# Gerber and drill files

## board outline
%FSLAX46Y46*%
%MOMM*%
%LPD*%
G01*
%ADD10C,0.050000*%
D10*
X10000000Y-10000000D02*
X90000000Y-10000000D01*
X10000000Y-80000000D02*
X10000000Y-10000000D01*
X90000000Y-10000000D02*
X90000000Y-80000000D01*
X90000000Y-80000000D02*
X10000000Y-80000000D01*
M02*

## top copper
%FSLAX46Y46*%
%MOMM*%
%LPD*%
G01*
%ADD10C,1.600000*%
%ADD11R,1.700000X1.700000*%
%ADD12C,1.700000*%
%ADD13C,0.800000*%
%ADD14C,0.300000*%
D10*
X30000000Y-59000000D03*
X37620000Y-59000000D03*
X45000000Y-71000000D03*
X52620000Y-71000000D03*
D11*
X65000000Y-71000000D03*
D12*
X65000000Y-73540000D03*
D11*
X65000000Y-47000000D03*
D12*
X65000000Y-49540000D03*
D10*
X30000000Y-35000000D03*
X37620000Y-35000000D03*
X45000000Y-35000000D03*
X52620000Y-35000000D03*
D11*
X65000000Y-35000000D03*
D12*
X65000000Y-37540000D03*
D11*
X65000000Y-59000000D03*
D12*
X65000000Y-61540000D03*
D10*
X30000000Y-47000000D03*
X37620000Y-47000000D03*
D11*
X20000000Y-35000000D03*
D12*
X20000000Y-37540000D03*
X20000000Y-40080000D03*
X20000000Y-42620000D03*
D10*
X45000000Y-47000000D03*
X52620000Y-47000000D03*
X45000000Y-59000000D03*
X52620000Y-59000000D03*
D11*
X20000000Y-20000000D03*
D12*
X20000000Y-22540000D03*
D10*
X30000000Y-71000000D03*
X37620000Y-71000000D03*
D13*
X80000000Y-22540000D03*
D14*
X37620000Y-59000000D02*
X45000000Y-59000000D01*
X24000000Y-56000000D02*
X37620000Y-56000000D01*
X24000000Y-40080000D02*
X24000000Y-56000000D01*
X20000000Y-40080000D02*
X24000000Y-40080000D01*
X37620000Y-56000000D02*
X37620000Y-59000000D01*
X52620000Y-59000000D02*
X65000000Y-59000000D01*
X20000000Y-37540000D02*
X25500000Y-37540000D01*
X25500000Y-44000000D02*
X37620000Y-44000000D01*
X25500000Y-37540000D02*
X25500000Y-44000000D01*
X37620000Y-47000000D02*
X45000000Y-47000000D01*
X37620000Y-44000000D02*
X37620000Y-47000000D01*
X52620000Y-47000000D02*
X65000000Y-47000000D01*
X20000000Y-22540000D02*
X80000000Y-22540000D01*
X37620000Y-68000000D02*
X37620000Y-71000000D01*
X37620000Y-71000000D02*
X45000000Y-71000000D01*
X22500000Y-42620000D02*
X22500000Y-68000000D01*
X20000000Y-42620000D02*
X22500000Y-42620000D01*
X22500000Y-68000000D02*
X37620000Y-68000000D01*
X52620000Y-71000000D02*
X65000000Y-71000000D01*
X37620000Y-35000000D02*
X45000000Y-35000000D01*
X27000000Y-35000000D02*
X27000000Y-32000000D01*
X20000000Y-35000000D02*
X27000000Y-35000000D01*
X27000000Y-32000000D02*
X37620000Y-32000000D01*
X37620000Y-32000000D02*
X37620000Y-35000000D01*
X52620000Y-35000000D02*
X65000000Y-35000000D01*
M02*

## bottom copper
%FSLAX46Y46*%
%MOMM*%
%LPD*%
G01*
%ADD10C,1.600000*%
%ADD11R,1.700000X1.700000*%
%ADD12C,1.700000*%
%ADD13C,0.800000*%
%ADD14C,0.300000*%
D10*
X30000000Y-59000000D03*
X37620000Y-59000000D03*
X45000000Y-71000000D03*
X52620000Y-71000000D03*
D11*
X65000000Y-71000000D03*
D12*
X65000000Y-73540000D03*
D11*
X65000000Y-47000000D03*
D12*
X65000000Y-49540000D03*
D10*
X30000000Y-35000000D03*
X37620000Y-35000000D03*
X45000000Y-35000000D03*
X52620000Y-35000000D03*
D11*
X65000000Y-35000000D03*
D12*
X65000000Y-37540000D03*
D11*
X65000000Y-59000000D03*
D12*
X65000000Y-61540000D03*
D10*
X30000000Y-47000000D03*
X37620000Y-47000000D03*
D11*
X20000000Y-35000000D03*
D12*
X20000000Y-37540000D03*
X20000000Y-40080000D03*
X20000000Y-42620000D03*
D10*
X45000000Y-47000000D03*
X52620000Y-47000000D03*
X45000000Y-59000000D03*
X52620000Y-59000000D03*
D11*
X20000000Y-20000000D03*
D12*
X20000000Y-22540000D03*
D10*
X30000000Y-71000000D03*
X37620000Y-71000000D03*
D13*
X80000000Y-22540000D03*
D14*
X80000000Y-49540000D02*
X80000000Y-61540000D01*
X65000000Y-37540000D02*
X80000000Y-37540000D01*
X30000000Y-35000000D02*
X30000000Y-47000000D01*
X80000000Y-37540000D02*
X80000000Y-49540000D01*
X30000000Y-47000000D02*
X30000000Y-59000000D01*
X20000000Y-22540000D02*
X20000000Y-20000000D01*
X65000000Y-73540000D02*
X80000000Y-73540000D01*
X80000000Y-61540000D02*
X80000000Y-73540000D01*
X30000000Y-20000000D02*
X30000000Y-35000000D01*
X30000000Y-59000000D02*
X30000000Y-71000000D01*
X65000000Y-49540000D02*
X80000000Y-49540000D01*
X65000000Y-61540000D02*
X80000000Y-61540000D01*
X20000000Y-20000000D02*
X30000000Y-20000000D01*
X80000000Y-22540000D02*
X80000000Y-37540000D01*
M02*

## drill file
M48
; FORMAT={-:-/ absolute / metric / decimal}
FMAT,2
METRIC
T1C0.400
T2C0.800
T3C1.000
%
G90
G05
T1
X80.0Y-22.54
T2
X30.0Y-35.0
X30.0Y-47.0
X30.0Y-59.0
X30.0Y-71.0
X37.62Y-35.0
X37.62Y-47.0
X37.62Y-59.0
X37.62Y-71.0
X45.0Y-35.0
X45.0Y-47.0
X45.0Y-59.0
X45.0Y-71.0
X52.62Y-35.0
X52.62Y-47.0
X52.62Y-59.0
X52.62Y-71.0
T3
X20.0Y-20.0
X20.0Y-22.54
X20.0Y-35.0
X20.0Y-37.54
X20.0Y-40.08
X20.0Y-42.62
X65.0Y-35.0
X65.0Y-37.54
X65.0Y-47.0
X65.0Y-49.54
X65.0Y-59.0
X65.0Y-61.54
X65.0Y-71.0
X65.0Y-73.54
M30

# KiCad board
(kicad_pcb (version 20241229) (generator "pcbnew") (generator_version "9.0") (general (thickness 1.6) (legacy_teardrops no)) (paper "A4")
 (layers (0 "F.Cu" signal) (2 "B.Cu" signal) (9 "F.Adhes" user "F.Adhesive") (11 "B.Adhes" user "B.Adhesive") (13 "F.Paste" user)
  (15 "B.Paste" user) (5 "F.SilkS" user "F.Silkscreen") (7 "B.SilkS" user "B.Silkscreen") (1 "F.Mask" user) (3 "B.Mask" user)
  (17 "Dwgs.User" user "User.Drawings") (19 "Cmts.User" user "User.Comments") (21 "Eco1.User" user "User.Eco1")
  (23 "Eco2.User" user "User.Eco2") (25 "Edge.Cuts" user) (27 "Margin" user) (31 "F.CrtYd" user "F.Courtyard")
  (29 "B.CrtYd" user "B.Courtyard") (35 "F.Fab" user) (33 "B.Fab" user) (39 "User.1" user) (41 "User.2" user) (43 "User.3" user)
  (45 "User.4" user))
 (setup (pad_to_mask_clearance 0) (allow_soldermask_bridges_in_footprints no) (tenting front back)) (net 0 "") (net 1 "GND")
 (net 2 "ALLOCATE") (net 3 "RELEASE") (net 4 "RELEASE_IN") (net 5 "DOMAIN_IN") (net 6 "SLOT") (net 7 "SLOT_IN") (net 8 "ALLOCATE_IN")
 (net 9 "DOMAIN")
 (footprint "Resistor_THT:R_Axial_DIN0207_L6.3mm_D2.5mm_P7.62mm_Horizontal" (layer "F.Cu") (at 30 59)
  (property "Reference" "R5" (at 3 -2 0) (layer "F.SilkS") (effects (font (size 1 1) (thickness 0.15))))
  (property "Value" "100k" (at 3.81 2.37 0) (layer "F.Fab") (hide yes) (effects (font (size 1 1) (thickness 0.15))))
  (pad "1" thru_hole circle (at 0 0) (size 1.6 1.6) (drill 0.8) (layers "*.Cu" "*.Mask") (remove_unused_layers no) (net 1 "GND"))
  (pad "2" thru_hole circle (at 7.62 0) (size 1.6 1.6) (drill 0.8) (layers "*.Cu" "*.Mask") (remove_unused_layers no) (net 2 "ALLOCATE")))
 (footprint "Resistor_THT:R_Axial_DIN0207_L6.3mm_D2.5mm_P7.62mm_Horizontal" (layer "F.Cu") (at 45 71)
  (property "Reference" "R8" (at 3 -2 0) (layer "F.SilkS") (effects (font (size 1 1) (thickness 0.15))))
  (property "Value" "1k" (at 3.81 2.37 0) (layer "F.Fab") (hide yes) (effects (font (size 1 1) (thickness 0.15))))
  (pad "1" thru_hole circle (at 0 0) (size 1.6 1.6) (drill 0.8) (layers "*.Cu" "*.Mask") (remove_unused_layers no) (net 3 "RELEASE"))
  (pad "2" thru_hole circle (at 7.62 0) (size 1.6 1.6) (drill 0.8) (layers "*.Cu" "*.Mask") (remove_unused_layers no) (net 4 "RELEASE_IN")))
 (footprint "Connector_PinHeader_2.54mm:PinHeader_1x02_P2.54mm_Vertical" (layer "F.Cu") (at 65 71)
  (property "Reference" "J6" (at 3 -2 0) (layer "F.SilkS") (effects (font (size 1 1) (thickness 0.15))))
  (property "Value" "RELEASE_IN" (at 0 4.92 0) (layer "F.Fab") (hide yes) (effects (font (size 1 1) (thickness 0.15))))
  (pad "1" thru_hole rect (at 0 0) (size 1.7 1.7) (drill 1) (layers "*.Cu" "*.Mask") (remove_unused_layers no) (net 4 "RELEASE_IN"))
  (pad "2" thru_hole circle (at 0 2.54) (size 1.7 1.7) (drill 1) (layers "*.Cu" "*.Mask") (remove_unused_layers no) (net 1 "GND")))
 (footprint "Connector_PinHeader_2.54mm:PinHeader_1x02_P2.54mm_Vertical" (layer "F.Cu") (at 65 47)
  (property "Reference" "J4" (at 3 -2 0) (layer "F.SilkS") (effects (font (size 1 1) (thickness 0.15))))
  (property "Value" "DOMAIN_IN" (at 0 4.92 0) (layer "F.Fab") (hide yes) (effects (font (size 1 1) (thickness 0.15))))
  (pad "1" thru_hole rect (at 0 0) (size 1.7 1.7) (drill 1) (layers "*.Cu" "*.Mask") (remove_unused_layers no) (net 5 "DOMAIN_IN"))
  (pad "2" thru_hole circle (at 0 2.54) (size 1.7 1.7) (drill 1) (layers "*.Cu" "*.Mask") (remove_unused_layers no) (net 1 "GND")))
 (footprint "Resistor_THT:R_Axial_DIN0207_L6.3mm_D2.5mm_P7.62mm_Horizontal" (layer "F.Cu") (at 30 35)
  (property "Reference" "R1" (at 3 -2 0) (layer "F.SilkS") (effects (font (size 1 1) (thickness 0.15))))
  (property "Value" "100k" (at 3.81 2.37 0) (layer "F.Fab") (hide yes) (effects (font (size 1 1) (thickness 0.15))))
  (pad "1" thru_hole circle (at 0 0) (size 1.6 1.6) (drill 0.8) (layers "*.Cu" "*.Mask") (remove_unused_layers no) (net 1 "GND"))
  (pad "2" thru_hole circle (at 7.62 0) (size 1.6 1.6) (drill 0.8) (layers "*.Cu" "*.Mask") (remove_unused_layers no) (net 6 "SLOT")))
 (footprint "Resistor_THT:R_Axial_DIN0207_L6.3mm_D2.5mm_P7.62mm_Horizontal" (layer "F.Cu") (at 45 35)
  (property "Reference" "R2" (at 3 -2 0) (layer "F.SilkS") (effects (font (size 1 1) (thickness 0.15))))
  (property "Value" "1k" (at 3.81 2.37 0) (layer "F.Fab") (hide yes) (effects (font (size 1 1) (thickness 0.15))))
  (pad "1" thru_hole circle (at 0 0) (size 1.6 1.6) (drill 0.8) (layers "*.Cu" "*.Mask") (remove_unused_layers no) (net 6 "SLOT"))
  (pad "2" thru_hole circle (at 7.62 0) (size 1.6 1.6) (drill 0.8) (layers "*.Cu" "*.Mask") (remove_unused_layers no) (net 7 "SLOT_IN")))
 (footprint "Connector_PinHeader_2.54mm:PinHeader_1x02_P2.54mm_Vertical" (layer "F.Cu") (at 65 35)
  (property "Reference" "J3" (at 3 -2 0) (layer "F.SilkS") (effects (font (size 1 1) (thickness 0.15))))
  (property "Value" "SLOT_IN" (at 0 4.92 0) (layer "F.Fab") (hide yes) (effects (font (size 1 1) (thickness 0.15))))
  (pad "1" thru_hole rect (at 0 0) (size 1.7 1.7) (drill 1) (layers "*.Cu" "*.Mask") (remove_unused_layers no) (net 7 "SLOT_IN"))
  (pad "2" thru_hole circle (at 0 2.54) (size 1.7 1.7) (drill 1) (layers "*.Cu" "*.Mask") (remove_unused_layers no) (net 1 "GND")))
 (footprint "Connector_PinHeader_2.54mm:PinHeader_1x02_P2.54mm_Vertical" (layer "F.Cu") (at 65 59)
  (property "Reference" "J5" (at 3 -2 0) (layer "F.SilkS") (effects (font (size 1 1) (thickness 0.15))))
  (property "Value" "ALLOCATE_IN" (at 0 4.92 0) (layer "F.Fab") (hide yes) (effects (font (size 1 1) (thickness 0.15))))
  (pad "1" thru_hole rect (at 0 0) (size 1.7 1.7) (drill 1) (layers "*.Cu" "*.Mask") (remove_unused_layers no) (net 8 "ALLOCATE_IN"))
  (pad "2" thru_hole circle (at 0 2.54) (size 1.7 1.7) (drill 1) (layers "*.Cu" "*.Mask") (remove_unused_layers no) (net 1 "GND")))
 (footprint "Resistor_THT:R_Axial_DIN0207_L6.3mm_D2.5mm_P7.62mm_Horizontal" (layer "F.Cu") (at 30 47)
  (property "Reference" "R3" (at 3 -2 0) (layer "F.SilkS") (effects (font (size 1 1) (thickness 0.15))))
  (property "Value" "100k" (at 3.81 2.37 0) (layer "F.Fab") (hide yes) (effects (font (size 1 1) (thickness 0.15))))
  (pad "1" thru_hole circle (at 0 0) (size 1.6 1.6) (drill 0.8) (layers "*.Cu" "*.Mask") (remove_unused_layers no) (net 1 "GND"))
  (pad "2" thru_hole circle (at 7.62 0) (size 1.6 1.6) (drill 0.8) (layers "*.Cu" "*.Mask") (remove_unused_layers no) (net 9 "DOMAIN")))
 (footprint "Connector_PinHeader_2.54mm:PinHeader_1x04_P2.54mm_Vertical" (layer "F.Cu") (at 20 35)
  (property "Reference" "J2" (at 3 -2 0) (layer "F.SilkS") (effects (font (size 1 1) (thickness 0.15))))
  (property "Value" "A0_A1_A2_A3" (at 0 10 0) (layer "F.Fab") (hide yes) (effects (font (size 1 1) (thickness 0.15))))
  (pad "1" thru_hole rect (at 0 0) (size 1.7 1.7) (drill 1) (layers "*.Cu" "*.Mask") (remove_unused_layers no) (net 6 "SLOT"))
  (pad "2" thru_hole circle (at 0 2.54) (size 1.7 1.7) (drill 1) (layers "*.Cu" "*.Mask") (remove_unused_layers no) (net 9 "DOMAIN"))
  (pad "3" thru_hole circle (at 0 5.08) (size 1.7 1.7) (drill 1) (layers "*.Cu" "*.Mask") (remove_unused_layers no) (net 2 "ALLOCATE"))
  (pad "4" thru_hole circle (at 0 7.62) (size 1.7 1.7) (drill 1) (layers "*.Cu" "*.Mask") (remove_unused_layers no) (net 3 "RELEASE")))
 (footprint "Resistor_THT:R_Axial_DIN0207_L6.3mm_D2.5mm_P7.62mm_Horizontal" (layer "F.Cu") (at 45 47)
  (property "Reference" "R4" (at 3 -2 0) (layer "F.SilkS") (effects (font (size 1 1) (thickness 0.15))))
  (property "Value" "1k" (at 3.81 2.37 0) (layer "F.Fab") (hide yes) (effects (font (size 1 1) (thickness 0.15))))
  (pad "1" thru_hole circle (at 0 0) (size 1.6 1.6) (drill 0.8) (layers "*.Cu" "*.Mask") (remove_unused_layers no) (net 9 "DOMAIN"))
  (pad "2" thru_hole circle (at 7.62 0) (size 1.6 1.6) (drill 0.8) (layers "*.Cu" "*.Mask") (remove_unused_layers no) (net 5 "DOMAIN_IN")))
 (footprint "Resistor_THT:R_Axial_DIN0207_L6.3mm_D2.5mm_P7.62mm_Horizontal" (layer "F.Cu") (at 45 59)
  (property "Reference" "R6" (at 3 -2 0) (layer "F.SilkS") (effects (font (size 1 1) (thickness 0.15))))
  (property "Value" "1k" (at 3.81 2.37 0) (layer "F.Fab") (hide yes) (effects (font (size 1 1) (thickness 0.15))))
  (pad "1" thru_hole circle (at 0 0) (size 1.6 1.6) (drill 0.8) (layers "*.Cu" "*.Mask") (remove_unused_layers no) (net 2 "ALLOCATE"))
  (pad "2" thru_hole circle (at 7.62 0) (size 1.6 1.6) (drill 0.8) (layers "*.Cu" "*.Mask") (remove_unused_layers no) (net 8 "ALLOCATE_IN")))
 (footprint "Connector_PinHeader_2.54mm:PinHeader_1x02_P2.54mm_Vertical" (layer "F.Cu") (at 20 20)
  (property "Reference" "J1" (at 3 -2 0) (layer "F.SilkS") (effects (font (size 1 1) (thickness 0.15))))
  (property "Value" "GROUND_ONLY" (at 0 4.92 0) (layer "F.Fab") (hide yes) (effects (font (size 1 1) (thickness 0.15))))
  (pad "1" thru_hole rect (at 0 0) (size 1.7 1.7) (drill 1) (layers "*.Cu" "*.Mask") (remove_unused_layers no) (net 1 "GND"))
  (pad "2" thru_hole circle (at 0 2.54) (size 1.7 1.7) (drill 1) (layers "*.Cu" "*.Mask") (remove_unused_layers no) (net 1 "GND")))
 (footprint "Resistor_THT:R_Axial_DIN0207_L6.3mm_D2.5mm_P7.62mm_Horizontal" (layer "F.Cu") (at 30 71)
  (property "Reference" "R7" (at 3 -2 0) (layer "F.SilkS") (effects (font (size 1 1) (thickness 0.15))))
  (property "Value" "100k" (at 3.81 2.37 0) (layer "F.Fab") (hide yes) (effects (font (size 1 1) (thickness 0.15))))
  (pad "1" thru_hole circle (at 0 0) (size 1.6 1.6) (drill 0.8) (layers "*.Cu" "*.Mask") (remove_unused_layers no) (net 1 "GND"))
  (pad "2" thru_hole circle (at 7.62 0) (size 1.6 1.6) (drill 0.8) (layers "*.Cu" "*.Mask") (remove_unused_layers no) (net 3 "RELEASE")))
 (gr_line (start 10 10) (end 90 10) (stroke (width 0.05) (type default)) (layer "Edge.Cuts"))
 (gr_line (start 10 80) (end 10 10) (stroke (width 0.05) (type default)) (layer "Edge.Cuts"))
 (gr_line (start 90 10) (end 90 80) (stroke (width 0.05) (type default)) (layer "Edge.Cuts"))
 (gr_line (start 90 80) (end 10 80) (stroke (width 0.05) (type default)) (layer "Edge.Cuts"))
 (segment (start 37.62 59) (end 45 59) (width 0.3) (layer "F.Cu") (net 2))
 (segment (start 24 56) (end 37.62 56) (width 0.3) (layer "F.Cu") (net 2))
 (segment (start 24 40.08) (end 24 56) (width 0.3) (layer "F.Cu") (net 2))
 (segment (start 20 40.08) (end 24 40.08) (width 0.3) (layer "F.Cu") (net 2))
 (segment (start 37.62 56) (end 37.62 59) (width 0.3) (layer "F.Cu") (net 2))
 (segment (start 52.62 59) (end 65 59) (width 0.3) (layer "F.Cu") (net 8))
 (segment (start 20 37.54) (end 25.5 37.54) (width 0.3) (layer "F.Cu") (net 9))
 (segment (start 25.5 44) (end 37.62 44) (width 0.3) (layer "F.Cu") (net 9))
 (segment (start 25.5 37.54) (end 25.5 44) (width 0.3) (layer "F.Cu") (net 9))
 (segment (start 37.62 47) (end 45 47) (width 0.3) (layer "F.Cu") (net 9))
 (segment (start 37.62 44) (end 37.62 47) (width 0.3) (layer "F.Cu") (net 9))
 (segment (start 52.62 47) (end 65 47) (width 0.3) (layer "F.Cu") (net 5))
 (segment (start 20 22.54) (end 80 22.54) (width 0.3) (layer "F.Cu") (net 1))
 (via (at 80 22.54) (size 0.8) (drill 0.4) (layers "F.Cu" "B.Cu") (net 1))
 (segment (start 80 49.54) (end 80 61.54) (width 0.3) (layer "B.Cu") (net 1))
 (segment (start 65 37.54) (end 80 37.54) (width 0.3) (layer "B.Cu") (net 1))
 (segment (start 30 35) (end 30 47) (width 0.3) (layer "B.Cu") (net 1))
 (segment (start 80 37.54) (end 80 49.54) (width 0.3) (layer "B.Cu") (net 1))
 (segment (start 30 47) (end 30 59) (width 0.3) (layer "B.Cu") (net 1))
 (segment (start 20 22.54) (end 20 20) (width 0.3) (layer "B.Cu") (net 1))
 (segment (start 65 73.54) (end 80 73.54) (width 0.3) (layer "B.Cu") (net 1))
 (segment (start 80 61.54) (end 80 73.54) (width 0.3) (layer "B.Cu") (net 1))
 (segment (start 30 20) (end 30 35) (width 0.3) (layer "B.Cu") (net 1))
 (segment (start 30 59) (end 30 71) (width 0.3) (layer "B.Cu") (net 1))
 (segment (start 65 49.54) (end 80 49.54) (width 0.3) (layer "B.Cu") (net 1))
 (segment (start 65 61.54) (end 80 61.54) (width 0.3) (layer "B.Cu") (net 1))
 (segment (start 20 20) (end 30 20) (width 0.3) (layer "B.Cu") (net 1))
 (segment (start 80 22.54) (end 80 37.54) (width 0.3) (layer "B.Cu") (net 1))
 (segment (start 37.62 68) (end 37.62 71) (width 0.3) (layer "F.Cu") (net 3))
 (segment (start 37.62 71) (end 45 71) (width 0.3) (layer "F.Cu") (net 3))
 (segment (start 22.5 42.62) (end 22.5 68) (width 0.3) (layer "F.Cu") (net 3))
 (segment (start 20 42.62) (end 22.5 42.62) (width 0.3) (layer "F.Cu") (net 3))
 (segment (start 22.5 68) (end 37.62 68) (width 0.3) (layer "F.Cu") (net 3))
 (segment (start 52.62 71) (end 65 71) (width 0.3) (layer "F.Cu") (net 4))
 (segment (start 37.62 35) (end 45 35) (width 0.3) (layer "F.Cu") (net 6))
 (segment (start 27 35) (end 27 32) (width 0.3) (layer "F.Cu") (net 6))
 (segment (start 20 35) (end 27 35) (width 0.3) (layer "F.Cu") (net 6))
 (segment (start 27 32) (end 37.62 32) (width 0.3) (layer "F.Cu") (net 6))
 (segment (start 37.62 32) (end 37.62 35) (width 0.3) (layer "F.Cu") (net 6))
 (segment (start 52.62 35) (end 65 35) (width 0.3) (layer "F.Cu") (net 7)))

